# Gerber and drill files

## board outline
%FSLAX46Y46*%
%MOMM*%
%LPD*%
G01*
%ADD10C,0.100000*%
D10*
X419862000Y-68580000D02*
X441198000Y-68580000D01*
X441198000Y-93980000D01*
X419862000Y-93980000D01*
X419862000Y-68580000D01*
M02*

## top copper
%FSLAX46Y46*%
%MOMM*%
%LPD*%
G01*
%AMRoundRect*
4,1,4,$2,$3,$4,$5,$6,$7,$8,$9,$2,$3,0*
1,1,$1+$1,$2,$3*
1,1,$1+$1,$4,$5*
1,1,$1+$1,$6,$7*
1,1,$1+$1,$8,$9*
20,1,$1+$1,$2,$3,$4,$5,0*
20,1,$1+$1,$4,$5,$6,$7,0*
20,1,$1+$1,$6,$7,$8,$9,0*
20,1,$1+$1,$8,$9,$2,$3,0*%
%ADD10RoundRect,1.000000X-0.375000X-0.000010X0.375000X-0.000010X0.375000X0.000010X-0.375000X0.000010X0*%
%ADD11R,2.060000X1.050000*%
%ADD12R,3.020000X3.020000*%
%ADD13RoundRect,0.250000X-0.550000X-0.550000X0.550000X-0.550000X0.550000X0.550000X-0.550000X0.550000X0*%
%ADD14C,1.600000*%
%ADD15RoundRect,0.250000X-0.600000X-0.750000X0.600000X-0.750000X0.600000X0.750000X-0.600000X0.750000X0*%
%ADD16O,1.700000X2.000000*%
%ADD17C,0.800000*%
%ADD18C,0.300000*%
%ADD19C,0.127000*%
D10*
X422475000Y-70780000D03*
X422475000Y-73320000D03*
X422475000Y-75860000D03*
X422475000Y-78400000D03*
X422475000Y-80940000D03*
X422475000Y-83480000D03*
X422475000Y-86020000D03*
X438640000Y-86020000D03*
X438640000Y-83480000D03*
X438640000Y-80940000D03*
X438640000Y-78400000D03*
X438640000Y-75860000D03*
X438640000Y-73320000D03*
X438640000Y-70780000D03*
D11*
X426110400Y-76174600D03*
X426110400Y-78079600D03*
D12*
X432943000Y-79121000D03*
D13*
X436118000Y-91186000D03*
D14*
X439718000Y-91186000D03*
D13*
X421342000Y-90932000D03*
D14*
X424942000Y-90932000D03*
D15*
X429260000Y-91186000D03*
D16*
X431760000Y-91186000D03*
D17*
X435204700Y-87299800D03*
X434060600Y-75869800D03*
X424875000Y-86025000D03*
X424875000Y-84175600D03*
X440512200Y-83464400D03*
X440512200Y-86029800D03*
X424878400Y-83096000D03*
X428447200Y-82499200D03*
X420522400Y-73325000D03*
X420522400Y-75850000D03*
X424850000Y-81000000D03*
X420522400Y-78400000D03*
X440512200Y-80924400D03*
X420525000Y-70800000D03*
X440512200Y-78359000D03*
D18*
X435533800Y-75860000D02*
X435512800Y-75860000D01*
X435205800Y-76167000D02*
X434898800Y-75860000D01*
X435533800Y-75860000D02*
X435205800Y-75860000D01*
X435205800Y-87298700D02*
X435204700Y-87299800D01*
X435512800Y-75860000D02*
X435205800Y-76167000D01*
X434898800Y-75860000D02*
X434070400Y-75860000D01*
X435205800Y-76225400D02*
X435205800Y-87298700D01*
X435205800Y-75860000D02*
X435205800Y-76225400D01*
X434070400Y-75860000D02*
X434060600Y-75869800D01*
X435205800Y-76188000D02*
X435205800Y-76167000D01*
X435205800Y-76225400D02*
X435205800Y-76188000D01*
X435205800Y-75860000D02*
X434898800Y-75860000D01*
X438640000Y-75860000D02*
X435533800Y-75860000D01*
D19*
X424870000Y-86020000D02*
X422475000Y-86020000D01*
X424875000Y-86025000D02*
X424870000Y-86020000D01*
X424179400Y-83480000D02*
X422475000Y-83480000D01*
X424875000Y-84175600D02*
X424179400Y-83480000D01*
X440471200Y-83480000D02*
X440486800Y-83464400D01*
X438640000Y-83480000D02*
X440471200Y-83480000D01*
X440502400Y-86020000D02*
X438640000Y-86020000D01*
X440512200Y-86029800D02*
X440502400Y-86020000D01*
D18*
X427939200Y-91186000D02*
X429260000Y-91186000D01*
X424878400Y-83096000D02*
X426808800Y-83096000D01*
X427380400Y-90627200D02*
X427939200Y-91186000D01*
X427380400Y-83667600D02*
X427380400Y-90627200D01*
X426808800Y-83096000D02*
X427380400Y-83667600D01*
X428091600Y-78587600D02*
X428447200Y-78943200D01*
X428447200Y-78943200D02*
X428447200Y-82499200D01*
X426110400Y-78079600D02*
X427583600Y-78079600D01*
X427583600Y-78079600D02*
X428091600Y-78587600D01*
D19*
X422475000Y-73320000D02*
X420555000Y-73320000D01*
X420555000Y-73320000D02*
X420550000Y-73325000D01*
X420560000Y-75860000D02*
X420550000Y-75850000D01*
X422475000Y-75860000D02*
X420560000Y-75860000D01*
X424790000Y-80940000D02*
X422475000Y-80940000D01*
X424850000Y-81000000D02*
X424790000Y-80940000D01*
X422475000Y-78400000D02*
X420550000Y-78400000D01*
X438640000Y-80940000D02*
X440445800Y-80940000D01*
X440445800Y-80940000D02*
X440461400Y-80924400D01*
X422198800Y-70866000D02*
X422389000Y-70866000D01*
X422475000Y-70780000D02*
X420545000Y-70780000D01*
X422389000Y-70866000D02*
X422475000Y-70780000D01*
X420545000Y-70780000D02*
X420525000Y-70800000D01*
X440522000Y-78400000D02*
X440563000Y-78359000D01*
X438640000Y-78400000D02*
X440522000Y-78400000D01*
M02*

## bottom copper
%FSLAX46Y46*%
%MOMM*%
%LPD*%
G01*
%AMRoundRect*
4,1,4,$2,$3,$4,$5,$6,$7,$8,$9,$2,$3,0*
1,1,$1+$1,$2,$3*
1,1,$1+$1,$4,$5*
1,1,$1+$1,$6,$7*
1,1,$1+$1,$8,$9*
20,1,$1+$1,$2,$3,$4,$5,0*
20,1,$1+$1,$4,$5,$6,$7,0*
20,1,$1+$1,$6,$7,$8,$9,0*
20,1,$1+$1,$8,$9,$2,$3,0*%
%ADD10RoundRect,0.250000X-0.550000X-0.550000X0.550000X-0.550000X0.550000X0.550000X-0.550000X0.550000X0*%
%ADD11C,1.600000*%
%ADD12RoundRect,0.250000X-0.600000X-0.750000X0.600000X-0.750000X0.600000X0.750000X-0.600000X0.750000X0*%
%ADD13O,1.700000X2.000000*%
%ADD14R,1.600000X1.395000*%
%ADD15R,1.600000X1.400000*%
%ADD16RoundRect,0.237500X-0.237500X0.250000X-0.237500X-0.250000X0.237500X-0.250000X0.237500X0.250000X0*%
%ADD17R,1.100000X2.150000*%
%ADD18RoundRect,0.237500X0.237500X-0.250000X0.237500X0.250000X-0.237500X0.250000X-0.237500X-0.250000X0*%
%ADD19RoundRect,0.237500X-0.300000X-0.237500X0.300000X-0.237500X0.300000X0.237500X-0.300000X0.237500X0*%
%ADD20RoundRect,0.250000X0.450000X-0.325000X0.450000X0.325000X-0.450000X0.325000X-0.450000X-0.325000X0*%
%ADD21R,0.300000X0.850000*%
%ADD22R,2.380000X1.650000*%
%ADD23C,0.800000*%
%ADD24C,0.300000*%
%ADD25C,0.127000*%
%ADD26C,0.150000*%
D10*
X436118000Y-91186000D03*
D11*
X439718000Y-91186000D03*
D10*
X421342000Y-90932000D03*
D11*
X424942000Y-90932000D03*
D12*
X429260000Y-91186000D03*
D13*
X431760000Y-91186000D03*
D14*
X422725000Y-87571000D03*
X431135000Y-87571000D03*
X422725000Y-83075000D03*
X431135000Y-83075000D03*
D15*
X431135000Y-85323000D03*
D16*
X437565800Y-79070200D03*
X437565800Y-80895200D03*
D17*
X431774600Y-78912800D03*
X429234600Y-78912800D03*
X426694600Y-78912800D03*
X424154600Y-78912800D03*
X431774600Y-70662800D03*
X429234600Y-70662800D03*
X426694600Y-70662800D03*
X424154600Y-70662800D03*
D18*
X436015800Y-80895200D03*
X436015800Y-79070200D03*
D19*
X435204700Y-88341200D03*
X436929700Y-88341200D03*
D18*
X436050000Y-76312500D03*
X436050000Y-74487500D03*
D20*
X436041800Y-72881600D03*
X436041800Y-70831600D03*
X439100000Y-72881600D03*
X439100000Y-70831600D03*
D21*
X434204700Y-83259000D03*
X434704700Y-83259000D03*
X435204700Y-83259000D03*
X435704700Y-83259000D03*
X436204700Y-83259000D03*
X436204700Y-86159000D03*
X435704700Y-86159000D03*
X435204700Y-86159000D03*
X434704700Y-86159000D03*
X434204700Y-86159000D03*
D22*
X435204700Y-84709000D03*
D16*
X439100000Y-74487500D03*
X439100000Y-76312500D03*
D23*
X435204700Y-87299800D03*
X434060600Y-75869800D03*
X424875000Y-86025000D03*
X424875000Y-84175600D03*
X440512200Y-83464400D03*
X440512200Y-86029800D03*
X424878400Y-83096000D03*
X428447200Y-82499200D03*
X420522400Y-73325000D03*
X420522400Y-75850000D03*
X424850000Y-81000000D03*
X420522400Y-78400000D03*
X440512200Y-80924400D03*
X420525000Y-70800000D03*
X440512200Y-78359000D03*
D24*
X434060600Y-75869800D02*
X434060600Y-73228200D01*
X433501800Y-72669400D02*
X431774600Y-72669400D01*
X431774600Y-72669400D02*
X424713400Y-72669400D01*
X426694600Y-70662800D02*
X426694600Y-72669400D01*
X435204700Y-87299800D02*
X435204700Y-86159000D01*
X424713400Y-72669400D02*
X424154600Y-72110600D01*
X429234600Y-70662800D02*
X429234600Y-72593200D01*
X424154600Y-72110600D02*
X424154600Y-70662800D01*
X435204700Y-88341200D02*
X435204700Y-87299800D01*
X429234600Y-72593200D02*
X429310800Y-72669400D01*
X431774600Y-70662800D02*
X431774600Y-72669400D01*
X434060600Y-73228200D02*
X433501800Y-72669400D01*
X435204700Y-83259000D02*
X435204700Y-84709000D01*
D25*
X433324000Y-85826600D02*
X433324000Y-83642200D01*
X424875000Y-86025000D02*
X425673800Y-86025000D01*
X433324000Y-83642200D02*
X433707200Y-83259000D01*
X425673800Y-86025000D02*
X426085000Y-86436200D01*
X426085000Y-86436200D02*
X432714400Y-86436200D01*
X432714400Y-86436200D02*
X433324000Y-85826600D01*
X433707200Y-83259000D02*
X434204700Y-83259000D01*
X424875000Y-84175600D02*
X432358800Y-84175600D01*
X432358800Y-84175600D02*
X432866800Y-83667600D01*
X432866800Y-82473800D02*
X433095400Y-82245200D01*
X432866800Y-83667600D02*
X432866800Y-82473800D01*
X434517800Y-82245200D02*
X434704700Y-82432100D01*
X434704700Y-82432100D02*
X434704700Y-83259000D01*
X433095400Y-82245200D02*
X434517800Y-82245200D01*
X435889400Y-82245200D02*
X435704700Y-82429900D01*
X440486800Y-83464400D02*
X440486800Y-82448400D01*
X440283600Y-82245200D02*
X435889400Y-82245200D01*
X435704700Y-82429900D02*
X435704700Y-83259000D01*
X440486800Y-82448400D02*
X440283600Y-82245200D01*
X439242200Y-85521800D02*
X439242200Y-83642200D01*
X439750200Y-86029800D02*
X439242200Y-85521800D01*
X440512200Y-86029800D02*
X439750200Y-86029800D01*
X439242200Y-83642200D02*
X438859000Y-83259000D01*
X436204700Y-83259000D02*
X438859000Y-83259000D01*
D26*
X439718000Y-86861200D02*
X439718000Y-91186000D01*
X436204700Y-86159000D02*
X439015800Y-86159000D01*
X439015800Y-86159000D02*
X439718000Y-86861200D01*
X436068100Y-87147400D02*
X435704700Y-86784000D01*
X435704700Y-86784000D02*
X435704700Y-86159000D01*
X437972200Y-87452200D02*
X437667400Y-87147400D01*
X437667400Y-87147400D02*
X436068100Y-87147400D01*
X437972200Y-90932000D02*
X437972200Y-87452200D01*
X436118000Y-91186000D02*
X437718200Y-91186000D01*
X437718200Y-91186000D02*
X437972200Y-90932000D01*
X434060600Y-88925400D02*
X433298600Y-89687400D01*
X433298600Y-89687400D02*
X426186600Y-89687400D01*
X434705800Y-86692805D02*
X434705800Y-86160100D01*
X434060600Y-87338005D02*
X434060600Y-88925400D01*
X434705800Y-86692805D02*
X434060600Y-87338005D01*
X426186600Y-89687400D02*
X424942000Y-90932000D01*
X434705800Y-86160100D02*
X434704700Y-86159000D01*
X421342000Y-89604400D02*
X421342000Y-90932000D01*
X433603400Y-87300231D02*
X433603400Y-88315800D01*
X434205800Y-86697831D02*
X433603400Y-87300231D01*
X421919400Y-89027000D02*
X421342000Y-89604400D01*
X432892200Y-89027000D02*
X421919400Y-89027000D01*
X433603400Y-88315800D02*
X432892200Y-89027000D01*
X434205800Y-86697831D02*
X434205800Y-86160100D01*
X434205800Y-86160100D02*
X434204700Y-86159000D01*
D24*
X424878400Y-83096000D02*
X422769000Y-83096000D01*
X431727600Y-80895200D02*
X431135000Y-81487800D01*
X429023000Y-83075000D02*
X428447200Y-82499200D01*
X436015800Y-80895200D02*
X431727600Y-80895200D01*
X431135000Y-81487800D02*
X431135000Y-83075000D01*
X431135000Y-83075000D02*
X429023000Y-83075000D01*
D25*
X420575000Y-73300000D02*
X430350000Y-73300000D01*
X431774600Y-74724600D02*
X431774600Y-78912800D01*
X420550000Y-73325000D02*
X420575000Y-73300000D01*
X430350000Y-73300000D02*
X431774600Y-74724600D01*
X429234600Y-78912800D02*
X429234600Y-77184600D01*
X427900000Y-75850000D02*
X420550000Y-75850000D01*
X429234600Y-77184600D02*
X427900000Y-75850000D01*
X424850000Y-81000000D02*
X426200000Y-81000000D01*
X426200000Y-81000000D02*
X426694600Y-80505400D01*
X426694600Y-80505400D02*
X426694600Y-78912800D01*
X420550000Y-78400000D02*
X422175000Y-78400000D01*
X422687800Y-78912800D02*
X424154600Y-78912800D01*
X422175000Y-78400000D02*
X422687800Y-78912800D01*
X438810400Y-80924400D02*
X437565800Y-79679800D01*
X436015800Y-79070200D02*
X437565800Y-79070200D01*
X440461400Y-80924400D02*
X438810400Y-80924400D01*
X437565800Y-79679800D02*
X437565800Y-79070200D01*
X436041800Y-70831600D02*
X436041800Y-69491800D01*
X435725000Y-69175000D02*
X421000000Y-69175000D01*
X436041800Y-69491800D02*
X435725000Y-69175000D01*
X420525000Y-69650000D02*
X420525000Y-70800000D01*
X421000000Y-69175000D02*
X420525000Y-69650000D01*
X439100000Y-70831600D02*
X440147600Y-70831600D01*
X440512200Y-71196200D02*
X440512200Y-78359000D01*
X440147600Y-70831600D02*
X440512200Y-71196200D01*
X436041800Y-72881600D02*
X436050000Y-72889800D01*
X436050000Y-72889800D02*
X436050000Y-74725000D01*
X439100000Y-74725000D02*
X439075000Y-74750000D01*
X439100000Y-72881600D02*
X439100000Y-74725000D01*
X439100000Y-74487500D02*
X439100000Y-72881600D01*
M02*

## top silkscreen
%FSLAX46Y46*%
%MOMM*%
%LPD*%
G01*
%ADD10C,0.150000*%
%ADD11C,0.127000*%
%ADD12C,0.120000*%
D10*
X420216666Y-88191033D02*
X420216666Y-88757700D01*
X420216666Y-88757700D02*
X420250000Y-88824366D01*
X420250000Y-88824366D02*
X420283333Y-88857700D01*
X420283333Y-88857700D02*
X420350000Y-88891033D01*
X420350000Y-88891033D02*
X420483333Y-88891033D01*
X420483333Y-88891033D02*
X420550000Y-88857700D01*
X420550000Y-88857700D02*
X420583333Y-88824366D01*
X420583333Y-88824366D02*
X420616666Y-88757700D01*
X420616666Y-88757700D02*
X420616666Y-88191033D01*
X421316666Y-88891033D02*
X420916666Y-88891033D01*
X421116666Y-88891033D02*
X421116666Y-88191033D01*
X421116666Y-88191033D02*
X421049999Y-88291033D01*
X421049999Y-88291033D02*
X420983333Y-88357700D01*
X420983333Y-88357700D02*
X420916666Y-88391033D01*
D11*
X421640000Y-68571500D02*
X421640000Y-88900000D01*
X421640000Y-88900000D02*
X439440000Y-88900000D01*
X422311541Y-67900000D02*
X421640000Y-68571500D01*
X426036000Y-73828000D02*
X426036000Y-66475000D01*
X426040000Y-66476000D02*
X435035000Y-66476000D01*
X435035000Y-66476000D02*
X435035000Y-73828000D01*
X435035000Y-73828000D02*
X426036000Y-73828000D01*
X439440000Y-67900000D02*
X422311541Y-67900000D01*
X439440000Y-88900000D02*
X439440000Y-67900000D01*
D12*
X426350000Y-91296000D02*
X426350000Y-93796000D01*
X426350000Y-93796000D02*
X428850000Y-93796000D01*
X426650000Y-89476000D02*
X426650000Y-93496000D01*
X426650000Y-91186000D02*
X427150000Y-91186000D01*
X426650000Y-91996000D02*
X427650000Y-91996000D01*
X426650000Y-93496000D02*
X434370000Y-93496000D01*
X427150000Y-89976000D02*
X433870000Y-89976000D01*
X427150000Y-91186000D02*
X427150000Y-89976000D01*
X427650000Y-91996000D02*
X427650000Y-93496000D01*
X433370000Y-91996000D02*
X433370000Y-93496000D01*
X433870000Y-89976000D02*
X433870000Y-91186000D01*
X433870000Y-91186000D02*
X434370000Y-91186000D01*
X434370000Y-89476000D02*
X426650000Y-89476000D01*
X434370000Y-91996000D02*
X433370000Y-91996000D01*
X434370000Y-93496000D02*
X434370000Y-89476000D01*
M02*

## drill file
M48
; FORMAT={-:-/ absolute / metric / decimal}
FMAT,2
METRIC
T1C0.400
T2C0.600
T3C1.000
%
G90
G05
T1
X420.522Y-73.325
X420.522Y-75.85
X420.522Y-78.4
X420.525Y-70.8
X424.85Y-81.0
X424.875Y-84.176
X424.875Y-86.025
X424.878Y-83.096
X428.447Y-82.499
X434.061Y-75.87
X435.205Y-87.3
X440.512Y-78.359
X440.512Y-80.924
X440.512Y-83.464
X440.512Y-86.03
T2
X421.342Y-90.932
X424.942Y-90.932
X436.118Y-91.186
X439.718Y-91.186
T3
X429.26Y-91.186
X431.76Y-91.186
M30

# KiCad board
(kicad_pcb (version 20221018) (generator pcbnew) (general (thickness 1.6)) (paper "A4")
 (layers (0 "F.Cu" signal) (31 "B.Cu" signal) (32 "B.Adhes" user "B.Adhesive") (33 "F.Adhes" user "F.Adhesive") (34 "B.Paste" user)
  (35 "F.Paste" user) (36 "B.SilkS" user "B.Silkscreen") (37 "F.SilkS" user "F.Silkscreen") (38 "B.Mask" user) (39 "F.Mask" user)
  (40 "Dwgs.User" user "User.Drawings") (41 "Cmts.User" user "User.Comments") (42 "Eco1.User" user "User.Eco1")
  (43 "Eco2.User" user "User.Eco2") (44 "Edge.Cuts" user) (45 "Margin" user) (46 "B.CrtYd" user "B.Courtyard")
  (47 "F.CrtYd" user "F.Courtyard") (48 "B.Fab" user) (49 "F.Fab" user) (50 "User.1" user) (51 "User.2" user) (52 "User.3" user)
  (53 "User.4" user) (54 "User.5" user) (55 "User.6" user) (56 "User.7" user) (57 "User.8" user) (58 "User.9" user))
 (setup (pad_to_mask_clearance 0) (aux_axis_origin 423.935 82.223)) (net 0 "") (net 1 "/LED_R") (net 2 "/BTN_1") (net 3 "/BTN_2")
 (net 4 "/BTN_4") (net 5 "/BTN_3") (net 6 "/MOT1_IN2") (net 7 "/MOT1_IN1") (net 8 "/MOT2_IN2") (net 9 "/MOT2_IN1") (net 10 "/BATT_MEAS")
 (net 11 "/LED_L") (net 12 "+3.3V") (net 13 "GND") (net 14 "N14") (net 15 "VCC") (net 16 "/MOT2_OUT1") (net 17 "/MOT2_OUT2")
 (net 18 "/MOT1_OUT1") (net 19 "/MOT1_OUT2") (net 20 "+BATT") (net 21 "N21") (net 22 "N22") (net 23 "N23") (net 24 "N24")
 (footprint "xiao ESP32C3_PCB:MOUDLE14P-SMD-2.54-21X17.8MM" (layer "F.Cu") (at 421.64 88.9)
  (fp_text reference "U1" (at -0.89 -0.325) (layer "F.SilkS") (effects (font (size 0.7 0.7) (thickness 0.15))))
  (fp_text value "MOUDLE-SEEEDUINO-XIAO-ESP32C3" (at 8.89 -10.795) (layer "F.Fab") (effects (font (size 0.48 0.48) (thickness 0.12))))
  (fp_line (start 0 -20.3285) (end 0 0) (stroke (width 0.127) (type solid)) (layer "F.SilkS"))
  (fp_line (start 0 0) (end 17.8 0) (stroke (width 0.127) (type solid)) (layer "F.SilkS"))
  (fp_line (start 0.671541 -21) (end 0 -20.3285) (stroke (width 0.127) (type solid)) (layer "F.SilkS"))
  (fp_line (start 4.396 -15.072) (end 4.396 -22.425) (stroke (width 0.127) (type solid)) (layer "F.SilkS"))
  (fp_line (start 4.4 -22.424) (end 13.395 -22.424) (stroke (width 0.127) (type solid)) (layer "F.SilkS"))
  (fp_line (start 13.395 -22.424) (end 13.395 -15.072) (stroke (width 0.127) (type solid)) (layer "F.SilkS"))
  (fp_line (start 13.395 -15.072) (end 4.396 -15.072) (stroke (width 0.127) (type solid)) (layer "F.SilkS"))
  (fp_line (start 17.8 -21) (end 0.671541 -21) (stroke (width 0.127) (type solid)) (layer "F.SilkS"))
  (fp_line (start 17.8 0) (end 17.8 -21) (stroke (width 0.127) (type solid)) (layer "F.SilkS"))
  (pad "1" smd roundrect (at 0.835 -18.12) (size 2.75 2) (layers "F.Cu" "F.Paste" "F.Mask") (roundrect_rratio 0.5) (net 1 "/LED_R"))
  (pad "2" smd roundrect (at 0.835 -15.58) (size 2.75 2) (layers "F.Cu" "F.Paste" "F.Mask") (roundrect_rratio 0.5) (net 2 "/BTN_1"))
  (pad "3" smd roundrect (at 0.835 -13.04) (size 2.75 2) (layers "F.Cu" "F.Paste" "F.Mask") (roundrect_rratio 0.5) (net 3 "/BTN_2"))
  (pad "4" smd roundrect (at 0.835 -10.5) (size 2.75 2) (layers "F.Cu" "F.Paste" "F.Mask") (roundrect_rratio 0.5) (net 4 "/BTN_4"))
  (pad "5" smd roundrect (at 0.835 -7.96) (size 2.75 2) (layers "F.Cu" "F.Paste" "F.Mask") (roundrect_rratio 0.5) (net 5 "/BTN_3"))
  (pad "6" smd roundrect (at 0.835 -5.42) (size 2.75 2) (layers "F.Cu" "F.Paste" "F.Mask") (roundrect_rratio 0.5) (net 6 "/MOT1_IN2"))
  (pad "7" smd roundrect (at 0.835 -2.88) (size 2.75 2) (layers "F.Cu" "F.Paste" "F.Mask") (roundrect_rratio 0.5) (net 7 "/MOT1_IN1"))
  (pad "8" smd roundrect (at 17 -2.88) (size 2.75 2) (layers "F.Cu" "F.Paste" "F.Mask") (roundrect_rratio 0.5) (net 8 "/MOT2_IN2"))
  (pad "9" smd roundrect (at 17 -5.42) (size 2.75 2) (layers "F.Cu" "F.Paste" "F.Mask") (roundrect_rratio 0.5) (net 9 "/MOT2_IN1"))
  (pad "10" smd roundrect (at 17 -7.96) (size 2.75 2) (layers "F.Cu" "F.Paste" "F.Mask") (roundrect_rratio 0.5) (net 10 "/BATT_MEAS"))
  (pad "11" smd roundrect (at 17 -10.5) (size 2.75 2) (layers "F.Cu" "F.Paste" "F.Mask") (roundrect_rratio 0.5) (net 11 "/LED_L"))
  (pad "12" smd roundrect (at 17 -13.04) (size 2.75 2) (layers "F.Cu" "F.Paste" "F.Mask") (roundrect_rratio 0.5) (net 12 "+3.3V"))
  (pad "13" smd roundrect (at 17 -15.58) (size 2.75 2) (layers "F.Cu" "F.Paste" "F.Mask") (roundrect_rratio 0.5) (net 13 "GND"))
  (pad "14" smd roundrect (at 17 -18.12) (size 2.75 2) (layers "F.Cu" "F.Paste" "F.Mask") (roundrect_rratio 0.5) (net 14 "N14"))
  (pad "15" smd rect (at 4.4704 -12.7254) (size 2.06 1.05) (layers "F.Cu" "F.Paste" "F.Mask") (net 13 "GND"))
  (pad "16" smd rect (at 4.4704 -10.8204) (size 2.06 1.05) (layers "F.Cu" "F.Paste" "F.Mask") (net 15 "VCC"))
  (pad "17" smd rect (at 11.303 -9.779) (size 3.02 3.02) (layers "F.Cu" "F.Paste" "F.Mask") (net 13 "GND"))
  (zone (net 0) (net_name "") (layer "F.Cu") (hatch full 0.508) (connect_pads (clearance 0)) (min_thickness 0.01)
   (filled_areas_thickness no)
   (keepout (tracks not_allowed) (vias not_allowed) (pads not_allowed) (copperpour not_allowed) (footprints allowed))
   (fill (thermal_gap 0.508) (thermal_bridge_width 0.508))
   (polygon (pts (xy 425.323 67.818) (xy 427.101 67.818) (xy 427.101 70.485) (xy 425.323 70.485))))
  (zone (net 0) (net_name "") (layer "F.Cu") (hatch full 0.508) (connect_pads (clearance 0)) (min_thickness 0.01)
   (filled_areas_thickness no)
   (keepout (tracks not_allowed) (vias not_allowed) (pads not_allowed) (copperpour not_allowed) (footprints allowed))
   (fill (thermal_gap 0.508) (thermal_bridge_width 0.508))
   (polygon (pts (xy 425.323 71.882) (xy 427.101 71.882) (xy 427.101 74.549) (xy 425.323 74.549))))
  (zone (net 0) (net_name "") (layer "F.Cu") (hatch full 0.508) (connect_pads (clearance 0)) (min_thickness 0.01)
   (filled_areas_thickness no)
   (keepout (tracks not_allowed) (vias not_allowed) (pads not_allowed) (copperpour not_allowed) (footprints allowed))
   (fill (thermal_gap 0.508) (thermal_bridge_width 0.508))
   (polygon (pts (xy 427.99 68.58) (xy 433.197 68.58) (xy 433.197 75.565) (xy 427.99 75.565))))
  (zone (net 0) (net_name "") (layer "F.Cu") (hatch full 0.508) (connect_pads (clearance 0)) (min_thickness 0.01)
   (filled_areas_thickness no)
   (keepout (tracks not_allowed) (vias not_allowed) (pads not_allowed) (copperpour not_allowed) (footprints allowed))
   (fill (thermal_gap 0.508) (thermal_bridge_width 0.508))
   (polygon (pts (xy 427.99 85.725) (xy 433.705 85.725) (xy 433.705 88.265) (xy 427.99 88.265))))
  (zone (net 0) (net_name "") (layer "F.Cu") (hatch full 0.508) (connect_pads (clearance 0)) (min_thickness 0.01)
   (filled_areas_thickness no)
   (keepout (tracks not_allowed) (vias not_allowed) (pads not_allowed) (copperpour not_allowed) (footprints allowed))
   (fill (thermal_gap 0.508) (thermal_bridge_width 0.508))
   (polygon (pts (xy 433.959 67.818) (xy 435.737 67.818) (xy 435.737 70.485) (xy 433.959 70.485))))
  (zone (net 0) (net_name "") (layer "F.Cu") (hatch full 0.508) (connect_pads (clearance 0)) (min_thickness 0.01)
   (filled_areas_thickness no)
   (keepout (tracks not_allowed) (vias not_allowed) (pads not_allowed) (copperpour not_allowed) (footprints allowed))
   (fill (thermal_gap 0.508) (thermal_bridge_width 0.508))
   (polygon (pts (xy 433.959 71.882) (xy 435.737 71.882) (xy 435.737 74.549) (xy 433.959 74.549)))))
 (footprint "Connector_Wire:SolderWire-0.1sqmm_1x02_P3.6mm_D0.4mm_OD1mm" (layer "F.Cu") (at 436.118 91.186)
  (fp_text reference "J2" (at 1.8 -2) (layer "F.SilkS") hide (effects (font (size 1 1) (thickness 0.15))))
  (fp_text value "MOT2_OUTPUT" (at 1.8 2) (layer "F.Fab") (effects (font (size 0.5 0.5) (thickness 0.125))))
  (pad "1" thru_hole roundrect (at 0 0) (size 1.6 1.6) (drill 0.6) (layers "*.Cu" "*.Mask") (roundrect_rratio 0.15625) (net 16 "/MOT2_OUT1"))
  (pad "2" thru_hole circle (at 3.6 0) (size 1.6 1.6) (drill 0.6) (layers "*.Cu" "*.Mask") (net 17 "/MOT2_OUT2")))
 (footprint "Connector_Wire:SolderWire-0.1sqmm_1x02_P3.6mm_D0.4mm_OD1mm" (layer "F.Cu") (at 421.342 90.932)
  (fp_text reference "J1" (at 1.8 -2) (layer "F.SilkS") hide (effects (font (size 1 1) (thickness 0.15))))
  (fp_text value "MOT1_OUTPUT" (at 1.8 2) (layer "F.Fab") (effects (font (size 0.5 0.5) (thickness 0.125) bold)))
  (pad "1" thru_hole roundrect (at 0 0) (size 1.6 1.6) (drill 0.6) (layers "*.Cu" "*.Mask") (roundrect_rratio 0.15625) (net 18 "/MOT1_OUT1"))
  (pad "2" thru_hole circle (at 3.6 0) (size 1.6 1.6) (drill 0.6) (layers "*.Cu" "*.Mask") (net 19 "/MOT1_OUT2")))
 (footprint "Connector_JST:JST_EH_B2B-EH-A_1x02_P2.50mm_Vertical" (layer "F.Cu") (at 429.26 91.186)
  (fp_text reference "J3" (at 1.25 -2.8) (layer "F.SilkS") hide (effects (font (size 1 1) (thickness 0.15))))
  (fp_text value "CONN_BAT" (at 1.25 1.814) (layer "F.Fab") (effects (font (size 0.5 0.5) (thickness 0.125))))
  (fp_line (start -2.91 0.11) (end -2.91 2.61) (stroke (width 0.12) (type solid)) (layer "F.SilkS"))
  (fp_line (start -2.91 2.61) (end -0.41 2.61) (stroke (width 0.12) (type solid)) (layer "F.SilkS"))
  (fp_line (start -2.61 -1.71) (end -2.61 2.31) (stroke (width 0.12) (type solid)) (layer "F.SilkS"))
  (fp_line (start -2.61 0) (end -2.11 0) (stroke (width 0.12) (type solid)) (layer "F.SilkS"))
  (fp_line (start -2.61 0.81) (end -1.61 0.81) (stroke (width 0.12) (type solid)) (layer "F.SilkS"))
  (fp_line (start -2.61 2.31) (end 5.11 2.31) (stroke (width 0.12) (type solid)) (layer "F.SilkS"))
  (fp_line (start -2.11 -1.21) (end 4.61 -1.21) (stroke (width 0.12) (type solid)) (layer "F.SilkS"))
  (fp_line (start -2.11 0) (end -2.11 -1.21) (stroke (width 0.12) (type solid)) (layer "F.SilkS"))
  (fp_line (start -1.61 0.81) (end -1.61 2.31) (stroke (width 0.12) (type solid)) (layer "F.SilkS"))
  (fp_line (start 4.11 0.81) (end 4.11 2.31) (stroke (width 0.12) (type solid)) (layer "F.SilkS"))
  (fp_line (start 4.61 -1.21) (end 4.61 0) (stroke (width 0.12) (type solid)) (layer "F.SilkS"))
  (fp_line (start 4.61 0) (end 5.11 0) (stroke (width 0.12) (type solid)) (layer "F.SilkS"))
  (fp_line (start 5.11 -1.71) (end -2.61 -1.71) (stroke (width 0.12) (type solid)) (layer "F.SilkS"))
  (fp_line (start 5.11 0.81) (end 4.11 0.81) (stroke (width 0.12) (type solid)) (layer "F.SilkS"))
  (fp_line (start 5.11 2.31) (end 5.11 -1.71) (stroke (width 0.12) (type solid)) (layer "F.SilkS"))
  (pad "1" thru_hole roundrect (at 0 0) (size 1.7 2) (drill 1) (layers "*.Cu" "*.Mask") (roundrect_rratio 0.147059) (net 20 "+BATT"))
  (pad "2" thru_hole oval (at 2.5 0) (size 1.7 2) (drill 1) (layers "*.Cu" "*.Mask") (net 13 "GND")))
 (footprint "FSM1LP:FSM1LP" (layer "B.Cu") (at 426.93 85.323)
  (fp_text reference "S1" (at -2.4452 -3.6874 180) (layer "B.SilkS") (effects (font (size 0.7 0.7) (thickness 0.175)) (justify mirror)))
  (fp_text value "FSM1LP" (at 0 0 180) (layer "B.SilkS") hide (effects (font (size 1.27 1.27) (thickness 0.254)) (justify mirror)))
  (pad "1" smd rect (at -4.205 2.248 270) (size 1.395 1.6) (layers "B.Cu" "B.Paste" "B.Mask") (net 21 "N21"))
  (pad "2" smd rect (at 4.205 2.248 270) (size 1.395 1.6) (layers "B.Cu" "B.Paste" "B.Mask") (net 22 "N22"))
  (pad "3" smd rect (at -4.205 -2.248 270) (size 1.395 1.6) (layers "B.Cu" "B.Paste" "B.Mask") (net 20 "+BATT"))
  (pad "4" smd rect (at 4.205 -2.248 270) (size 1.395 1.6) (layers "B.Cu" "B.Paste" "B.Mask") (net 15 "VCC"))
  (pad "5" smd rect (at 4.205 0 270) (size 1.4 1.6) (layers "B.Cu" "B.Paste" "B.Mask") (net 13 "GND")))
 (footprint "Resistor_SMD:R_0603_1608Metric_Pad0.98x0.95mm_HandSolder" (layer "B.Cu") (at 437.5658 79.9827 -90)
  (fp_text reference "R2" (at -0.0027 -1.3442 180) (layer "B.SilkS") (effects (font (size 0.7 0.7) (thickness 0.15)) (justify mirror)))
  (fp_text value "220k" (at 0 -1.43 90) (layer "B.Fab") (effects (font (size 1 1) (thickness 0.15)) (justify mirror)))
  (pad "1" smd roundrect (at -0.9125 0 270) (size 0.975 0.95) (layers "B.Cu" "B.Paste" "B.Mask") (roundrect_rratio 0.25)
   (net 10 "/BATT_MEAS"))
  (pad "2" smd roundrect (at 0.9125 0 270) (size 0.975 0.95) (layers "B.Cu" "B.Paste" "B.Mask") (roundrect_rratio 0.25) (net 13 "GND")))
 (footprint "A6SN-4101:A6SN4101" (layer "B.Cu") (at 427.9646 74.7878 180)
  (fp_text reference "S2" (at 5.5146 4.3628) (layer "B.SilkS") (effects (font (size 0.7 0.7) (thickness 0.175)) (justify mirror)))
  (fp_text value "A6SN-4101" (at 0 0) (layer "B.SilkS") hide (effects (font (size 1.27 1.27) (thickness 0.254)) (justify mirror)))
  (pad "A1" smd rect (at -3.81 -4.125 180) (size 1.1 2.15) (layers "B.Cu" "B.Paste" "B.Mask") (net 2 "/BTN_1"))
  (pad "A2" smd rect (at -1.27 -4.125 180) (size 1.1 2.15) (layers "B.Cu" "B.Paste" "B.Mask") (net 3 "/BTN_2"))
  (pad "A3" smd rect (at 1.27 -4.125 180) (size 1.1 2.15) (layers "B.Cu" "B.Paste" "B.Mask") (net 5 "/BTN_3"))
  (pad "A4" smd rect (at 3.81 -4.125 180) (size 1.1 2.15) (layers "B.Cu" "B.Paste" "B.Mask") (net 4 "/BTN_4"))
  (pad "B1" smd rect (at -3.81 4.125 180) (size 1.1 2.15) (layers "B.Cu" "B.Paste" "B.Mask") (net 12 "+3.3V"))
  (pad "B2" smd rect (at -1.27 4.125 180) (size 1.1 2.15) (layers "B.Cu" "B.Paste" "B.Mask") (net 12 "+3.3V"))
  (pad "B3" smd rect (at 1.27 4.125 180) (size 1.1 2.15) (layers "B.Cu" "B.Paste" "B.Mask") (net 12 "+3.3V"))
  (pad "B4" smd rect (at 3.81 4.125 180) (size 1.1 2.15) (layers "B.Cu" "B.Paste" "B.Mask") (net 12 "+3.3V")))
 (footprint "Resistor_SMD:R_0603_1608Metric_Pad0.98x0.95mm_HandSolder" (layer "B.Cu") (at 436.0158 79.9827 90)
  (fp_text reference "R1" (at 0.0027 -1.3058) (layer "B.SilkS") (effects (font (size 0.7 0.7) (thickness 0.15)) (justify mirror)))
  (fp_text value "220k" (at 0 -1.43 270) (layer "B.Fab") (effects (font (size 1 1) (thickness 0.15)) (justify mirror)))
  (pad "1" smd roundrect (at -0.9125 0 90) (size 0.975 0.95) (layers "B.Cu" "B.Paste" "B.Mask") (roundrect_rratio 0.25) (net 15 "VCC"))
  (pad "2" smd roundrect (at 0.9125 0 90) (size 0.975 0.95) (layers "B.Cu" "B.Paste" "B.Mask") (roundrect_rratio 0.25) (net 10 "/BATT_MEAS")))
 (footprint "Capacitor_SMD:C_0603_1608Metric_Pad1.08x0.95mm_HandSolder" (layer "B.Cu") (at 436.0672 88.3412)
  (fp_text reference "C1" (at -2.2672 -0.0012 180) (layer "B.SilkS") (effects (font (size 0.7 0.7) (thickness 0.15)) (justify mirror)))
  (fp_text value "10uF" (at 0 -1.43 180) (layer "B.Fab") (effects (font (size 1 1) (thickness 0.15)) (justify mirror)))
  (pad "1" smd roundrect (at -0.8625 0) (size 1.075 0.95) (layers "B.Cu" "B.Paste" "B.Mask") (roundrect_rratio 0.25) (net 12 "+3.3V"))
  (pad "2" smd roundrect (at 0.8625 0) (size 1.075 0.95) (layers "B.Cu" "B.Paste" "B.Mask") (roundrect_rratio 0.25) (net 13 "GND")))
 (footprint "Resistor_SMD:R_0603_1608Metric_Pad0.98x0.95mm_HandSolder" (layer "B.Cu") (at 436.05 75.4 90)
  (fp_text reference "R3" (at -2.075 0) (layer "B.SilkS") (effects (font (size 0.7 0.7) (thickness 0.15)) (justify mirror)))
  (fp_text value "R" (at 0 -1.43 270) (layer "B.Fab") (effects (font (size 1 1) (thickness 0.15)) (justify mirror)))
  (pad "1" smd roundrect (at -0.9125 0 90) (size 0.975 0.95) (layers "B.Cu" "B.Paste" "B.Mask") (roundrect_rratio 0.25) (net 13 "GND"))
  (pad "2" smd roundrect (at 0.9125 0 90) (size 0.975 0.95) (layers "B.Cu" "B.Paste" "B.Mask") (roundrect_rratio 0.25) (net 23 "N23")))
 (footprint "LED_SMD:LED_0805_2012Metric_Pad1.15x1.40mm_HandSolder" (layer "B.Cu") (at 436.0418 71.8566 90)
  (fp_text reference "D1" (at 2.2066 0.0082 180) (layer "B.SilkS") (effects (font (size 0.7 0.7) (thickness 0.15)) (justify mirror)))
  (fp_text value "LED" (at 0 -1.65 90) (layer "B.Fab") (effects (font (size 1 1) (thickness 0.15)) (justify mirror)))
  (pad "1" smd roundrect (at -1.025 0 90) (size 1.15 1.4) (layers "B.Cu" "B.Paste" "B.Mask") (roundrect_rratio 0.217391) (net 23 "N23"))
  (pad "2" smd roundrect (at 1.025 0 90) (size 1.15 1.4) (layers "B.Cu" "B.Paste" "B.Mask") (roundrect_rratio 0.217391) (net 1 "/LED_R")))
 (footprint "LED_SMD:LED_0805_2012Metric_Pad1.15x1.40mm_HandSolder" (layer "B.Cu") (at 439.1 71.8566 90)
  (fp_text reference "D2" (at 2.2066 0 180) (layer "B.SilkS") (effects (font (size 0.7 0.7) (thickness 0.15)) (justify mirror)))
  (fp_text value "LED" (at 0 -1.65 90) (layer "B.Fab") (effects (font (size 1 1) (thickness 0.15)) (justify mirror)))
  (pad "1" smd roundrect (at -1.025 0 90) (size 1.15 1.4) (layers "B.Cu" "B.Paste" "B.Mask") (roundrect_rratio 0.217391) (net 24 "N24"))
  (pad "2" smd roundrect (at 1.025 0 90) (size 1.15 1.4) (layers "B.Cu" "B.Paste" "B.Mask") (roundrect_rratio 0.217391) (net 11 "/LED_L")))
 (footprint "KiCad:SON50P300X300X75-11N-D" (layer "B.Cu") (at 435.2047 84.709 -90)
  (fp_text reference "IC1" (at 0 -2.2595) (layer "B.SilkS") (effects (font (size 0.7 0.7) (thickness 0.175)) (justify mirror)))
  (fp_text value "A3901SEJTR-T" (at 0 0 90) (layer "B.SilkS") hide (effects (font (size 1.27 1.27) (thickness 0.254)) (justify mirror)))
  (pad "1" smd rect (at -1.45 1 180) (size 0.3 0.85) (layers "B.Cu" "B.Paste" "B.Mask") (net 7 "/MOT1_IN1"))
  (pad "2" smd rect (at -1.45 0.5 180) (size 0.3 0.85) (layers "B.Cu" "B.Paste" "B.Mask") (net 6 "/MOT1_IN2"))
  (pad "3" smd rect (at -1.45 0 180) (size 0.3 0.85) (layers "B.Cu" "B.Paste" "B.Mask") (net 13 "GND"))
  (pad "4" smd rect (at -1.45 -0.5 180) (size 0.3 0.85) (layers "B.Cu" "B.Paste" "B.Mask") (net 9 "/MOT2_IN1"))
  (pad "5" smd rect (at -1.45 -1 180) (size 0.3 0.85) (layers "B.Cu" "B.Paste" "B.Mask") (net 8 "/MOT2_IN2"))
  (pad "6" smd rect (at 1.45 -1 180) (size 0.3 0.85) (layers "B.Cu" "B.Paste" "B.Mask") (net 17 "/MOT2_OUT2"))
  (pad "7" smd rect (at 1.45 -0.5 180) (size 0.3 0.85) (layers "B.Cu" "B.Paste" "B.Mask") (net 16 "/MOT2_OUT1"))
  (pad "8" smd rect (at 1.45 0 180) (size 0.3 0.85) (layers "B.Cu" "B.Paste" "B.Mask") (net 12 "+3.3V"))
  (pad "9" smd rect (at 1.45 0.5 180) (size 0.3 0.85) (layers "B.Cu" "B.Paste" "B.Mask") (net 19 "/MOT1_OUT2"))
  (pad "10" smd rect (at 1.45 1 180) (size 0.3 0.85) (layers "B.Cu" "B.Paste" "B.Mask") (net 18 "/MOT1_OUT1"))
  (pad "11" smd rect (at 0 0 270) (size 1.65 2.38) (layers "B.Cu" "B.Paste" "B.Mask") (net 13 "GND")))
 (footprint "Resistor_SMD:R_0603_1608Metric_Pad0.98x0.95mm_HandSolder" (layer "B.Cu") (at 439.1 75.4 -90)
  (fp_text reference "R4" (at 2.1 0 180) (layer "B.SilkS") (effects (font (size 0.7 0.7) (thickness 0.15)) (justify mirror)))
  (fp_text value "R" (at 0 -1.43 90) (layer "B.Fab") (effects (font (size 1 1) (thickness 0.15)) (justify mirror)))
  (pad "1" smd roundrect (at -0.9125 0 270) (size 0.975 0.95) (layers "B.Cu" "B.Paste" "B.Mask") (roundrect_rratio 0.25) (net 24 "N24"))
  (pad "2" smd roundrect (at 0.9125 0 270) (size 0.975 0.95) (layers "B.Cu" "B.Paste" "B.Mask") (roundrect_rratio 0.25) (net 13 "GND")))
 (gr_rect (start 419.862 68.58) (end 441.198 93.98) (stroke (width 0.1) (type default)) (fill none) (layer "Edge.Cuts"))
 (segment (start 435.5338 75.86) (end 435.5128 75.86) (width 0.3) (layer "F.Cu") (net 12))
 (segment (start 435.2058 76.167) (end 434.8988 75.86) (width 0.3) (layer "F.Cu") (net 12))
 (segment (start 435.5338 75.86) (end 435.2058 75.86) (width 0.3) (layer "F.Cu") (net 12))
 (segment (start 435.2058 87.2987) (end 435.2047 87.2998) (width 0.3) (layer "F.Cu") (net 12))
 (segment (start 435.5128 75.86) (end 435.2058 76.167) (width 0.3) (layer "F.Cu") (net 12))
 (segment (start 434.8988 75.86) (end 434.0704 75.86) (width 0.3) (layer "F.Cu") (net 12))
 (segment (start 435.2058 76.2254) (end 435.2058 87.2987) (width 0.3) (layer "F.Cu") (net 12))
 (segment (start 435.2058 75.86) (end 435.2058 76.2254) (width 0.3) (layer "F.Cu") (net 12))
 (segment (start 434.0704 75.86) (end 434.0606 75.8698) (width 0.3) (layer "F.Cu") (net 12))
 (segment (start 435.2058 76.188) (end 435.2058 76.167) (width 0.3) (layer "F.Cu") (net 12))
 (segment (start 435.2058 76.2254) (end 435.2058 76.188) (width 0.3) (layer "F.Cu") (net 12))
 (segment (start 435.2058 75.86) (end 434.8988 75.86) (width 0.3) (layer "F.Cu") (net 12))
 (segment (start 438.64 75.86) (end 435.5338 75.86) (width 0.3) (layer "F.Cu") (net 12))
 (via (at 435.2047 87.2998) (size 0.8) (drill 0.4) (layers "F.Cu" "B.Cu") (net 12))
 (via (at 434.0606 75.8698) (size 0.8) (drill 0.4) (layers "F.Cu" "B.Cu") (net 12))
 (segment (start 434.0606 75.8698) (end 434.0606 73.2282) (width 0.3) (layer "B.Cu") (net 12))
 (segment (start 433.5018 72.6694) (end 431.7746 72.6694) (width 0.3) (layer "B.Cu") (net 12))
 (segment (start 431.7746 72.6694) (end 424.7134 72.6694) (width 0.3) (layer "B.Cu") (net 12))
 (segment (start 426.6946 70.6628) (end 426.6946 72.6694) (width 0.3) (layer "B.Cu") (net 12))
 (segment (start 435.2047 87.2998) (end 435.2047 86.159) (width 0.3) (layer "B.Cu") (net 12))
 (segment (start 424.7134 72.6694) (end 424.1546 72.1106) (width 0.3) (layer "B.Cu") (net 12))
 (segment (start 429.2346 70.6628) (end 429.2346 72.5932) (width 0.3) (layer "B.Cu") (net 12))
 (segment (start 424.1546 72.1106) (end 424.1546 70.6628) (width 0.3) (layer "B.Cu") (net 12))
 (segment (start 435.2047 88.3412) (end 435.2047 87.2998) (width 0.3) (layer "B.Cu") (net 12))
 (segment (start 429.2346 72.5932) (end 429.3108 72.6694) (width 0.3) (layer "B.Cu") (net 12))
 (segment (start 431.7746 70.6628) (end 431.7746 72.6694) (width 0.3) (layer "B.Cu") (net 12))
 (segment (start 434.0606 73.2282) (end 433.5018 72.6694) (width 0.3) (layer "B.Cu") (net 12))
 (segment (start 435.2047 83.259) (end 435.2047 84.709) (width 0.3) (layer "B.Cu") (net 13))
 (segment (start 424.87 86.02) (end 422.475 86.02) (width 0.127) (layer "F.Cu") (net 7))
 (segment (start 424.875 86.025) (end 424.87 86.02) (width 0.127) (layer "F.Cu") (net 7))
 (via (at 424.875 86.025) (size 0.8) (drill 0.4) (layers "F.Cu" "B.Cu") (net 7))
 (segment (start 433.324 85.8266) (end 433.324 83.6422) (width 0.127) (layer "B.Cu") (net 7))
 (segment (start 424.875 86.025) (end 425.6738 86.025) (width 0.127) (layer "B.Cu") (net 7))
 (segment (start 433.324 83.6422) (end 433.7072 83.259) (width 0.127) (layer "B.Cu") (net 7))
 (segment (start 425.6738 86.025) (end 426.085 86.4362) (width 0.127) (layer "B.Cu") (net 7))
 (segment (start 426.085 86.4362) (end 432.7144 86.4362) (width 0.127) (layer "B.Cu") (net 7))
 (segment (start 432.7144 86.4362) (end 433.324 85.8266) (width 0.127) (layer "B.Cu") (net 7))
 (segment (start 433.7072 83.259) (end 434.2047 83.259) (width 0.127) (layer "B.Cu") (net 7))
 (segment (start 424.1794 83.48) (end 422.475 83.48) (width 0.127) (layer "F.Cu") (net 6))
 (segment (start 424.875 84.1756) (end 424.1794 83.48) (width 0.127) (layer "F.Cu") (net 6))
 (via (at 424.875 84.1756) (size 0.8) (drill 0.4) (layers "F.Cu" "B.Cu") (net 6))
 (segment (start 424.875 84.1756) (end 432.3588 84.1756) (width 0.127) (layer "B.Cu") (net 6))
 (segment (start 432.3588 84.1756) (end 432.8668 83.6676) (width 0.127) (layer "B.Cu") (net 6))
 (segment (start 432.8668 82.4738) (end 433.0954 82.2452) (width 0.127) (layer "B.Cu") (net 6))
 (segment (start 432.8668 83.6676) (end 432.8668 82.4738) (width 0.127) (layer "B.Cu") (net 6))
 (segment (start 434.5178 82.2452) (end 434.7047 82.4321) (width 0.127) (layer "B.Cu") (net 6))
 (segment (start 434.7047 82.4321) (end 434.7047 83.259) (width 0.127) (layer "B.Cu") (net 6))
 (segment (start 433.0954 82.2452) (end 434.5178 82.2452) (width 0.127) (layer "B.Cu") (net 6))
 (segment (start 440.4712 83.48) (end 440.4868 83.4644) (width 0.127) (layer "F.Cu") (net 9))
 (segment (start 438.64 83.48) (end 440.4712 83.48) (width 0.127) (layer "F.Cu") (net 9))
 (via (at 440.5122 83.4644) (size 0.8) (drill 0.4) (layers "F.Cu" "B.Cu") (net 9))
 (segment (start 435.8894 82.2452) (end 435.7047 82.4299) (width 0.127) (layer "B.Cu") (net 9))
 (segment (start 440.4868 83.4644) (end 440.4868 82.4484) (width 0.127) (layer "B.Cu") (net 9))
 (segment (start 440.2836 82.2452) (end 435.8894 82.2452) (width 0.127) (layer "B.Cu") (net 9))
 (segment (start 435.7047 82.4299) (end 435.7047 83.259) (width 0.127) (layer "B.Cu") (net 9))
 (segment (start 440.4868 82.4484) (end 440.2836 82.2452) (width 0.127) (layer "B.Cu") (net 9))
 (segment (start 440.5024 86.02) (end 438.64 86.02) (width 0.127) (layer "F.Cu") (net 8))
 (segment (start 440.5122 86.0298) (end 440.5024 86.02) (width 0.127) (layer "F.Cu") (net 8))
 (via (at 440.5122 86.0298) (size 0.8) (drill 0.4) (layers "F.Cu" "B.Cu") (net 8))
 (segment (start 439.2422 85.5218) (end 439.2422 83.6422) (width 0.127) (layer "B.Cu") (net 8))
 (segment (start 439.7502 86.0298) (end 439.2422 85.5218) (width 0.127) (layer "B.Cu") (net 8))
 (segment (start 440.5122 86.0298) (end 439.7502 86.0298) (width 0.127) (layer "B.Cu") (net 8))
 (segment (start 439.2422 83.6422) (end 438.859 83.259) (width 0.127) (layer "B.Cu") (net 8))
 (segment (start 436.2047 83.259) (end 438.859 83.259) (width 0.127) (layer "B.Cu") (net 8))
 (segment (start 439.718 86.8612) (end 439.718 91.186) (width 0.15) (layer "B.Cu") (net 17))
 (segment (start 436.2047 86.159) (end 439.0158 86.159) (width 0.15) (layer "B.Cu") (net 17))
 (segment (start 439.0158 86.159) (end 439.718 86.8612) (width 0.15) (layer "B.Cu") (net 17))
 (segment (start 436.0681 87.1474) (end 435.7047 86.784) (width 0.15) (layer "B.Cu") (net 16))
 (segment (start 435.7047 86.784) (end 435.7047 86.159) (width 0.15) (layer "B.Cu") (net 16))
 (segment (start 437.9722 87.4522) (end 437.6674 87.1474) (width 0.15) (layer "B.Cu") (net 16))
 (segment (start 437.6674 87.1474) (end 436.0681 87.1474) (width 0.15) (layer "B.Cu") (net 16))
 (segment (start 437.9722 90.932) (end 437.9722 87.4522) (width 0.15) (layer "B.Cu") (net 16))
 (segment (start 436.118 91.186) (end 437.7182 91.186) (width 0.15) (layer "B.Cu") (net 16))
 (segment (start 437.7182 91.186) (end 437.9722 90.932) (width 0.15) (layer "B.Cu") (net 16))
 (segment (start 434.0606 88.9254) (end 433.2986 89.6874) (width 0.15) (layer "B.Cu") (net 19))
 (segment (start 433.2986 89.6874) (end 426.1866 89.6874) (width 0.15) (layer "B.Cu") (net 19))
 (segment (start 434.7058 86.692805) (end 434.7058 86.1601) (width 0.15) (layer "B.Cu") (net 19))
 (segment (start 434.0606 87.338005) (end 434.0606 88.9254) (width 0.15) (layer "B.Cu") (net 19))
 (segment (start 434.7058 86.692805) (end 434.0606 87.338005) (width 0.15) (layer "B.Cu") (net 19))
 (segment (start 426.1866 89.6874) (end 424.942 90.932) (width 0.15) (layer "B.Cu") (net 19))
 (segment (start 434.7058 86.1601) (end 434.7047 86.159) (width 0.15) (layer "B.Cu") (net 19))
 (segment (start 421.342 89.6044) (end 421.342 90.932) (width 0.15) (layer "B.Cu") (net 18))
 (segment (start 433.6034 87.300231) (end 433.6034 88.3158) (width 0.15) (layer "B.Cu") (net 18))
 (segment (start 434.2058 86.697831) (end 433.6034 87.300231) (width 0.15) (layer "B.Cu") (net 18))
 (segment (start 421.9194 89.027) (end 421.342 89.6044) (width 0.15) (layer "B.Cu") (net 18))
 (segment (start 432.8922 89.027) (end 421.9194 89.027) (width 0.15) (layer "B.Cu") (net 18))
 (segment (start 433.6034 88.3158) (end 432.8922 89.027) (width 0.15) (layer "B.Cu") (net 18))
 (segment (start 434.2058 86.697831) (end 434.2058 86.1601) (width 0.15) (layer "B.Cu") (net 18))
 (segment (start 434.2058 86.1601) (end 434.2047 86.159) (width 0.15) (layer "B.Cu") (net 18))
 (segment (start 427.9392 91.186) (end 429.26 91.186) (width 0.3) (layer "F.Cu") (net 20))
 (segment (start 424.8784 83.096) (end 426.8088 83.096) (width 0.3) (layer "F.Cu") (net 20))
 (segment (start 427.3804 90.6272) (end 427.9392 91.186) (width 0.3) (layer "F.Cu") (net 20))
 (segment (start 427.3804 83.6676) (end 427.3804 90.6272) (width 0.3) (layer "F.Cu") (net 20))
 (segment (start 426.8088 83.096) (end 427.3804 83.6676) (width 0.3) (layer "F.Cu") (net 20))
 (via (at 424.8784 83.096) (size 0.8) (drill 0.4) (layers "F.Cu" "B.Cu") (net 20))
 (segment (start 424.8784 83.096) (end 422.769 83.096) (width 0.3) (layer "B.Cu") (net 20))
 (segment (start 428.0916 78.5876) (end 428.4472 78.9432) (width 0.3) (layer "F.Cu") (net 15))
 (segment (start 428.4472 78.9432) (end 428.4472 82.4992) (width 0.3) (layer "F.Cu") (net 15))
 (segment (start 426.1104 78.0796) (end 427.5836 78.0796) (width 0.3) (layer "F.Cu") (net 15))
 (segment (start 427.5836 78.0796) (end 428.0916 78.5876) (width 0.3) (layer "F.Cu") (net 15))
 (via (at 428.4472 82.4992) (size 0.8) (drill 0.4) (layers "F.Cu" "B.Cu") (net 15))
 (segment (start 431.7276 80.8952) (end 431.135 81.4878) (width 0.3) (layer "B.Cu") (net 15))
 (segment (start 429.023 83.075) (end 428.4472 82.4992) (width 0.3) (layer "B.Cu") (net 15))
 (segment (start 436.0158 80.8952) (end 431.7276 80.8952) (width 0.3) (layer "B.Cu") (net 15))
 (segment (start 431.135 81.4878) (end 431.135 83.075) (width 0.3) (layer "B.Cu") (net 15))
 (segment (start 431.135 83.075) (end 429.023 83.075) (width 0.3) (layer "B.Cu") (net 15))
 (segment (start 422.475 73.32) (end 420.555 73.32) (width 0.127) (layer "F.Cu") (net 2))
 (segment (start 420.555 73.32) (end 420.55 73.325) (width 0.127) (layer "F.Cu") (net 2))
 (via (at 420.5224 73.325) (size 0.8) (drill 0.4) (layers "F.Cu" "B.Cu") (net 2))
 (segment (start 420.575 73.3) (end 430.35 73.3) (width 0.127) (layer "B.Cu") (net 2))
 (segment (start 431.7746 74.7246) (end 431.7746 78.9128) (width 0.127) (layer "B.Cu") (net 2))
 (segment (start 420.55 73.325) (end 420.575 73.3) (width 0.127) (layer "B.Cu") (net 2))
 (segment (start 430.35 73.3) (end 431.7746 74.7246) (width 0.127) (layer "B.Cu") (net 2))
 (segment (start 420.56 75.86) (end 420.55 75.85) (width 0.127) (layer "F.Cu") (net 3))
 (segment (start 422.475 75.86) (end 420.56 75.86) (width 0.127) (layer "F.Cu") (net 3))
 (via (at 420.5224 75.85) (size 0.8) (drill 0.4) (layers "F.Cu" "B.Cu") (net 3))
 (segment (start 429.2346 78.9128) (end 429.2346 77.1846) (width 0.127) (layer "B.Cu") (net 3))
 (segment (start 427.9 75.85) (end 420.55 75.85) (width 0.127) (layer "B.Cu") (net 3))
 (segment (start 429.2346 77.1846) (end 427.9 75.85) (width 0.127) (layer "B.Cu") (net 3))
 (segment (start 424.79 80.94) (end 422.475 80.94) (width 0.127) (layer "F.Cu") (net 5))
 (segment (start 424.85 81) (end 424.79 80.94) (width 0.127) (layer "F.Cu") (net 5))
 (via (at 424.85 81) (size 0.8) (drill 0.4) (layers "F.Cu" "B.Cu") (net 5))
 (segment (start 424.85 81) (end 426.2 81) (width 0.127) (layer "B.Cu") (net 5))
 (segment (start 426.2 81) (end 426.6946 80.5054) (width 0.127) (layer "B.Cu") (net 5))
 (segment (start 426.6946 80.5054) (end 426.6946 78.9128) (width 0.127) (layer "B.Cu") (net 5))
 (segment (start 422.475 78.4) (end 420.55 78.4) (width 0.127) (layer "F.Cu") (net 4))
 (via (at 420.5224 78.4) (size 0.8) (drill 0.4) (layers "F.Cu" "B.Cu") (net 4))
 (segment (start 420.55 78.4) (end 422.175 78.4) (width 0.127) (layer "B.Cu") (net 4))
 (segment (start 422.6878 78.9128) (end 424.1546 78.9128) (width 0.127) (layer "B.Cu") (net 4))
 (segment (start 422.175 78.4) (end 422.6878 78.9128) (width 0.127) (layer "B.Cu") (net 4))
 (segment (start 438.64 80.94) (end 440.4458 80.94) (width 0.127) (layer "F.Cu") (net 10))
 (segment (start 440.4458 80.94) (end 440.4614 80.9244) (width 0.127) (layer "F.Cu") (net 10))
 (via (at 440.5122 80.9244) (size 0.8) (drill 0.4) (layers "F.Cu" "B.Cu") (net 10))
 (segment (start 438.8104 80.9244) (end 437.5658 79.6798) (width 0.127) (layer "B.Cu") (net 10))
 (segment (start 436.0158 79.0702) (end 437.5658 79.0702) (width 0.127) (layer "B.Cu") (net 10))
 (segment (start 440.4614 80.9244) (end 438.8104 80.9244) (width 0.127) (layer "B.Cu") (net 10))
 (segment (start 437.5658 79.6798) (end 437.5658 79.0702) (width 0.127) (layer "B.Cu") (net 10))
 (segment (start 422.1988 70.866) (end 422.389 70.866) (width 0.127) (layer "F.Cu") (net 1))
 (segment (start 422.475 70.78) (end 420.545 70.78) (width 0.127) (layer "F.Cu") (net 1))
 (segment (start 422.389 70.866) (end 422.475 70.78) (width 0.127) (layer "F.Cu") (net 1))
 (segment (start 420.545 70.78) (end 420.525 70.8) (width 0.127) (layer "F.Cu") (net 1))
 (via (at 420.525 70.8) (size 0.8) (drill 0.4) (layers "F.Cu" "B.Cu") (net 1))
 (segment (start 436.0418 70.8316) (end 436.0418 69.4918) (width 0.127) (layer "B.Cu") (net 1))
 (segment (start 435.725 69.175) (end 421 69.175) (width 0.127) (layer "B.Cu") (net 1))
 (segment (start 436.0418 69.4918) (end 435.725 69.175) (width 0.127) (layer "B.Cu") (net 1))
 (segment (start 420.525 69.65) (end 420.525 70.8) (width 0.127) (layer "B.Cu") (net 1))
 (segment (start 421 69.175) (end 420.525 69.65) (width 0.127) (layer "B.Cu") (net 1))
 (segment (start 440.522 78.4) (end 440.563 78.359) (width 0.127) (layer "F.Cu") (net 11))
 (segment (start 438.64 78.4) (end 440.522 78.4) (width 0.127) (layer "F.Cu") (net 11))
 (via (at 440.5122 78.359) (size 0.8) (drill 0.4) (layers "F.Cu" "B.Cu") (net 11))
 (segment (start 439.1 70.8316) (end 440.1476 70.8316) (width 0.127) (layer "B.Cu") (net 11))
 (segment (start 440.5122 71.1962) (end 440.5122 78.359) (width 0.127) (layer "B.Cu") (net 11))
 (segment (start 440.1476 70.8316) (end 440.5122 71.1962) (width 0.127) (layer "B.Cu") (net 11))
 (segment (start 436.0418 72.8816) (end 436.05 72.8898) (width 0.127) (layer "B.Cu") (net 23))
 (segment (start 436.05 72.8898) (end 436.05 74.725) (width 0.127) (layer "B.Cu") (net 23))
 (segment (start 439.1 74.725) (end 439.075 74.75) (width 0.127) (layer "B.Cu") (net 24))
 (segment (start 439.1 72.8816) (end 439.1 74.725) (width 0.127) (layer "B.Cu") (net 24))
 (segment (start 439.1 74.4875) (end 439.1 72.8816) (width 0.127) (layer "B.Cu") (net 24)))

